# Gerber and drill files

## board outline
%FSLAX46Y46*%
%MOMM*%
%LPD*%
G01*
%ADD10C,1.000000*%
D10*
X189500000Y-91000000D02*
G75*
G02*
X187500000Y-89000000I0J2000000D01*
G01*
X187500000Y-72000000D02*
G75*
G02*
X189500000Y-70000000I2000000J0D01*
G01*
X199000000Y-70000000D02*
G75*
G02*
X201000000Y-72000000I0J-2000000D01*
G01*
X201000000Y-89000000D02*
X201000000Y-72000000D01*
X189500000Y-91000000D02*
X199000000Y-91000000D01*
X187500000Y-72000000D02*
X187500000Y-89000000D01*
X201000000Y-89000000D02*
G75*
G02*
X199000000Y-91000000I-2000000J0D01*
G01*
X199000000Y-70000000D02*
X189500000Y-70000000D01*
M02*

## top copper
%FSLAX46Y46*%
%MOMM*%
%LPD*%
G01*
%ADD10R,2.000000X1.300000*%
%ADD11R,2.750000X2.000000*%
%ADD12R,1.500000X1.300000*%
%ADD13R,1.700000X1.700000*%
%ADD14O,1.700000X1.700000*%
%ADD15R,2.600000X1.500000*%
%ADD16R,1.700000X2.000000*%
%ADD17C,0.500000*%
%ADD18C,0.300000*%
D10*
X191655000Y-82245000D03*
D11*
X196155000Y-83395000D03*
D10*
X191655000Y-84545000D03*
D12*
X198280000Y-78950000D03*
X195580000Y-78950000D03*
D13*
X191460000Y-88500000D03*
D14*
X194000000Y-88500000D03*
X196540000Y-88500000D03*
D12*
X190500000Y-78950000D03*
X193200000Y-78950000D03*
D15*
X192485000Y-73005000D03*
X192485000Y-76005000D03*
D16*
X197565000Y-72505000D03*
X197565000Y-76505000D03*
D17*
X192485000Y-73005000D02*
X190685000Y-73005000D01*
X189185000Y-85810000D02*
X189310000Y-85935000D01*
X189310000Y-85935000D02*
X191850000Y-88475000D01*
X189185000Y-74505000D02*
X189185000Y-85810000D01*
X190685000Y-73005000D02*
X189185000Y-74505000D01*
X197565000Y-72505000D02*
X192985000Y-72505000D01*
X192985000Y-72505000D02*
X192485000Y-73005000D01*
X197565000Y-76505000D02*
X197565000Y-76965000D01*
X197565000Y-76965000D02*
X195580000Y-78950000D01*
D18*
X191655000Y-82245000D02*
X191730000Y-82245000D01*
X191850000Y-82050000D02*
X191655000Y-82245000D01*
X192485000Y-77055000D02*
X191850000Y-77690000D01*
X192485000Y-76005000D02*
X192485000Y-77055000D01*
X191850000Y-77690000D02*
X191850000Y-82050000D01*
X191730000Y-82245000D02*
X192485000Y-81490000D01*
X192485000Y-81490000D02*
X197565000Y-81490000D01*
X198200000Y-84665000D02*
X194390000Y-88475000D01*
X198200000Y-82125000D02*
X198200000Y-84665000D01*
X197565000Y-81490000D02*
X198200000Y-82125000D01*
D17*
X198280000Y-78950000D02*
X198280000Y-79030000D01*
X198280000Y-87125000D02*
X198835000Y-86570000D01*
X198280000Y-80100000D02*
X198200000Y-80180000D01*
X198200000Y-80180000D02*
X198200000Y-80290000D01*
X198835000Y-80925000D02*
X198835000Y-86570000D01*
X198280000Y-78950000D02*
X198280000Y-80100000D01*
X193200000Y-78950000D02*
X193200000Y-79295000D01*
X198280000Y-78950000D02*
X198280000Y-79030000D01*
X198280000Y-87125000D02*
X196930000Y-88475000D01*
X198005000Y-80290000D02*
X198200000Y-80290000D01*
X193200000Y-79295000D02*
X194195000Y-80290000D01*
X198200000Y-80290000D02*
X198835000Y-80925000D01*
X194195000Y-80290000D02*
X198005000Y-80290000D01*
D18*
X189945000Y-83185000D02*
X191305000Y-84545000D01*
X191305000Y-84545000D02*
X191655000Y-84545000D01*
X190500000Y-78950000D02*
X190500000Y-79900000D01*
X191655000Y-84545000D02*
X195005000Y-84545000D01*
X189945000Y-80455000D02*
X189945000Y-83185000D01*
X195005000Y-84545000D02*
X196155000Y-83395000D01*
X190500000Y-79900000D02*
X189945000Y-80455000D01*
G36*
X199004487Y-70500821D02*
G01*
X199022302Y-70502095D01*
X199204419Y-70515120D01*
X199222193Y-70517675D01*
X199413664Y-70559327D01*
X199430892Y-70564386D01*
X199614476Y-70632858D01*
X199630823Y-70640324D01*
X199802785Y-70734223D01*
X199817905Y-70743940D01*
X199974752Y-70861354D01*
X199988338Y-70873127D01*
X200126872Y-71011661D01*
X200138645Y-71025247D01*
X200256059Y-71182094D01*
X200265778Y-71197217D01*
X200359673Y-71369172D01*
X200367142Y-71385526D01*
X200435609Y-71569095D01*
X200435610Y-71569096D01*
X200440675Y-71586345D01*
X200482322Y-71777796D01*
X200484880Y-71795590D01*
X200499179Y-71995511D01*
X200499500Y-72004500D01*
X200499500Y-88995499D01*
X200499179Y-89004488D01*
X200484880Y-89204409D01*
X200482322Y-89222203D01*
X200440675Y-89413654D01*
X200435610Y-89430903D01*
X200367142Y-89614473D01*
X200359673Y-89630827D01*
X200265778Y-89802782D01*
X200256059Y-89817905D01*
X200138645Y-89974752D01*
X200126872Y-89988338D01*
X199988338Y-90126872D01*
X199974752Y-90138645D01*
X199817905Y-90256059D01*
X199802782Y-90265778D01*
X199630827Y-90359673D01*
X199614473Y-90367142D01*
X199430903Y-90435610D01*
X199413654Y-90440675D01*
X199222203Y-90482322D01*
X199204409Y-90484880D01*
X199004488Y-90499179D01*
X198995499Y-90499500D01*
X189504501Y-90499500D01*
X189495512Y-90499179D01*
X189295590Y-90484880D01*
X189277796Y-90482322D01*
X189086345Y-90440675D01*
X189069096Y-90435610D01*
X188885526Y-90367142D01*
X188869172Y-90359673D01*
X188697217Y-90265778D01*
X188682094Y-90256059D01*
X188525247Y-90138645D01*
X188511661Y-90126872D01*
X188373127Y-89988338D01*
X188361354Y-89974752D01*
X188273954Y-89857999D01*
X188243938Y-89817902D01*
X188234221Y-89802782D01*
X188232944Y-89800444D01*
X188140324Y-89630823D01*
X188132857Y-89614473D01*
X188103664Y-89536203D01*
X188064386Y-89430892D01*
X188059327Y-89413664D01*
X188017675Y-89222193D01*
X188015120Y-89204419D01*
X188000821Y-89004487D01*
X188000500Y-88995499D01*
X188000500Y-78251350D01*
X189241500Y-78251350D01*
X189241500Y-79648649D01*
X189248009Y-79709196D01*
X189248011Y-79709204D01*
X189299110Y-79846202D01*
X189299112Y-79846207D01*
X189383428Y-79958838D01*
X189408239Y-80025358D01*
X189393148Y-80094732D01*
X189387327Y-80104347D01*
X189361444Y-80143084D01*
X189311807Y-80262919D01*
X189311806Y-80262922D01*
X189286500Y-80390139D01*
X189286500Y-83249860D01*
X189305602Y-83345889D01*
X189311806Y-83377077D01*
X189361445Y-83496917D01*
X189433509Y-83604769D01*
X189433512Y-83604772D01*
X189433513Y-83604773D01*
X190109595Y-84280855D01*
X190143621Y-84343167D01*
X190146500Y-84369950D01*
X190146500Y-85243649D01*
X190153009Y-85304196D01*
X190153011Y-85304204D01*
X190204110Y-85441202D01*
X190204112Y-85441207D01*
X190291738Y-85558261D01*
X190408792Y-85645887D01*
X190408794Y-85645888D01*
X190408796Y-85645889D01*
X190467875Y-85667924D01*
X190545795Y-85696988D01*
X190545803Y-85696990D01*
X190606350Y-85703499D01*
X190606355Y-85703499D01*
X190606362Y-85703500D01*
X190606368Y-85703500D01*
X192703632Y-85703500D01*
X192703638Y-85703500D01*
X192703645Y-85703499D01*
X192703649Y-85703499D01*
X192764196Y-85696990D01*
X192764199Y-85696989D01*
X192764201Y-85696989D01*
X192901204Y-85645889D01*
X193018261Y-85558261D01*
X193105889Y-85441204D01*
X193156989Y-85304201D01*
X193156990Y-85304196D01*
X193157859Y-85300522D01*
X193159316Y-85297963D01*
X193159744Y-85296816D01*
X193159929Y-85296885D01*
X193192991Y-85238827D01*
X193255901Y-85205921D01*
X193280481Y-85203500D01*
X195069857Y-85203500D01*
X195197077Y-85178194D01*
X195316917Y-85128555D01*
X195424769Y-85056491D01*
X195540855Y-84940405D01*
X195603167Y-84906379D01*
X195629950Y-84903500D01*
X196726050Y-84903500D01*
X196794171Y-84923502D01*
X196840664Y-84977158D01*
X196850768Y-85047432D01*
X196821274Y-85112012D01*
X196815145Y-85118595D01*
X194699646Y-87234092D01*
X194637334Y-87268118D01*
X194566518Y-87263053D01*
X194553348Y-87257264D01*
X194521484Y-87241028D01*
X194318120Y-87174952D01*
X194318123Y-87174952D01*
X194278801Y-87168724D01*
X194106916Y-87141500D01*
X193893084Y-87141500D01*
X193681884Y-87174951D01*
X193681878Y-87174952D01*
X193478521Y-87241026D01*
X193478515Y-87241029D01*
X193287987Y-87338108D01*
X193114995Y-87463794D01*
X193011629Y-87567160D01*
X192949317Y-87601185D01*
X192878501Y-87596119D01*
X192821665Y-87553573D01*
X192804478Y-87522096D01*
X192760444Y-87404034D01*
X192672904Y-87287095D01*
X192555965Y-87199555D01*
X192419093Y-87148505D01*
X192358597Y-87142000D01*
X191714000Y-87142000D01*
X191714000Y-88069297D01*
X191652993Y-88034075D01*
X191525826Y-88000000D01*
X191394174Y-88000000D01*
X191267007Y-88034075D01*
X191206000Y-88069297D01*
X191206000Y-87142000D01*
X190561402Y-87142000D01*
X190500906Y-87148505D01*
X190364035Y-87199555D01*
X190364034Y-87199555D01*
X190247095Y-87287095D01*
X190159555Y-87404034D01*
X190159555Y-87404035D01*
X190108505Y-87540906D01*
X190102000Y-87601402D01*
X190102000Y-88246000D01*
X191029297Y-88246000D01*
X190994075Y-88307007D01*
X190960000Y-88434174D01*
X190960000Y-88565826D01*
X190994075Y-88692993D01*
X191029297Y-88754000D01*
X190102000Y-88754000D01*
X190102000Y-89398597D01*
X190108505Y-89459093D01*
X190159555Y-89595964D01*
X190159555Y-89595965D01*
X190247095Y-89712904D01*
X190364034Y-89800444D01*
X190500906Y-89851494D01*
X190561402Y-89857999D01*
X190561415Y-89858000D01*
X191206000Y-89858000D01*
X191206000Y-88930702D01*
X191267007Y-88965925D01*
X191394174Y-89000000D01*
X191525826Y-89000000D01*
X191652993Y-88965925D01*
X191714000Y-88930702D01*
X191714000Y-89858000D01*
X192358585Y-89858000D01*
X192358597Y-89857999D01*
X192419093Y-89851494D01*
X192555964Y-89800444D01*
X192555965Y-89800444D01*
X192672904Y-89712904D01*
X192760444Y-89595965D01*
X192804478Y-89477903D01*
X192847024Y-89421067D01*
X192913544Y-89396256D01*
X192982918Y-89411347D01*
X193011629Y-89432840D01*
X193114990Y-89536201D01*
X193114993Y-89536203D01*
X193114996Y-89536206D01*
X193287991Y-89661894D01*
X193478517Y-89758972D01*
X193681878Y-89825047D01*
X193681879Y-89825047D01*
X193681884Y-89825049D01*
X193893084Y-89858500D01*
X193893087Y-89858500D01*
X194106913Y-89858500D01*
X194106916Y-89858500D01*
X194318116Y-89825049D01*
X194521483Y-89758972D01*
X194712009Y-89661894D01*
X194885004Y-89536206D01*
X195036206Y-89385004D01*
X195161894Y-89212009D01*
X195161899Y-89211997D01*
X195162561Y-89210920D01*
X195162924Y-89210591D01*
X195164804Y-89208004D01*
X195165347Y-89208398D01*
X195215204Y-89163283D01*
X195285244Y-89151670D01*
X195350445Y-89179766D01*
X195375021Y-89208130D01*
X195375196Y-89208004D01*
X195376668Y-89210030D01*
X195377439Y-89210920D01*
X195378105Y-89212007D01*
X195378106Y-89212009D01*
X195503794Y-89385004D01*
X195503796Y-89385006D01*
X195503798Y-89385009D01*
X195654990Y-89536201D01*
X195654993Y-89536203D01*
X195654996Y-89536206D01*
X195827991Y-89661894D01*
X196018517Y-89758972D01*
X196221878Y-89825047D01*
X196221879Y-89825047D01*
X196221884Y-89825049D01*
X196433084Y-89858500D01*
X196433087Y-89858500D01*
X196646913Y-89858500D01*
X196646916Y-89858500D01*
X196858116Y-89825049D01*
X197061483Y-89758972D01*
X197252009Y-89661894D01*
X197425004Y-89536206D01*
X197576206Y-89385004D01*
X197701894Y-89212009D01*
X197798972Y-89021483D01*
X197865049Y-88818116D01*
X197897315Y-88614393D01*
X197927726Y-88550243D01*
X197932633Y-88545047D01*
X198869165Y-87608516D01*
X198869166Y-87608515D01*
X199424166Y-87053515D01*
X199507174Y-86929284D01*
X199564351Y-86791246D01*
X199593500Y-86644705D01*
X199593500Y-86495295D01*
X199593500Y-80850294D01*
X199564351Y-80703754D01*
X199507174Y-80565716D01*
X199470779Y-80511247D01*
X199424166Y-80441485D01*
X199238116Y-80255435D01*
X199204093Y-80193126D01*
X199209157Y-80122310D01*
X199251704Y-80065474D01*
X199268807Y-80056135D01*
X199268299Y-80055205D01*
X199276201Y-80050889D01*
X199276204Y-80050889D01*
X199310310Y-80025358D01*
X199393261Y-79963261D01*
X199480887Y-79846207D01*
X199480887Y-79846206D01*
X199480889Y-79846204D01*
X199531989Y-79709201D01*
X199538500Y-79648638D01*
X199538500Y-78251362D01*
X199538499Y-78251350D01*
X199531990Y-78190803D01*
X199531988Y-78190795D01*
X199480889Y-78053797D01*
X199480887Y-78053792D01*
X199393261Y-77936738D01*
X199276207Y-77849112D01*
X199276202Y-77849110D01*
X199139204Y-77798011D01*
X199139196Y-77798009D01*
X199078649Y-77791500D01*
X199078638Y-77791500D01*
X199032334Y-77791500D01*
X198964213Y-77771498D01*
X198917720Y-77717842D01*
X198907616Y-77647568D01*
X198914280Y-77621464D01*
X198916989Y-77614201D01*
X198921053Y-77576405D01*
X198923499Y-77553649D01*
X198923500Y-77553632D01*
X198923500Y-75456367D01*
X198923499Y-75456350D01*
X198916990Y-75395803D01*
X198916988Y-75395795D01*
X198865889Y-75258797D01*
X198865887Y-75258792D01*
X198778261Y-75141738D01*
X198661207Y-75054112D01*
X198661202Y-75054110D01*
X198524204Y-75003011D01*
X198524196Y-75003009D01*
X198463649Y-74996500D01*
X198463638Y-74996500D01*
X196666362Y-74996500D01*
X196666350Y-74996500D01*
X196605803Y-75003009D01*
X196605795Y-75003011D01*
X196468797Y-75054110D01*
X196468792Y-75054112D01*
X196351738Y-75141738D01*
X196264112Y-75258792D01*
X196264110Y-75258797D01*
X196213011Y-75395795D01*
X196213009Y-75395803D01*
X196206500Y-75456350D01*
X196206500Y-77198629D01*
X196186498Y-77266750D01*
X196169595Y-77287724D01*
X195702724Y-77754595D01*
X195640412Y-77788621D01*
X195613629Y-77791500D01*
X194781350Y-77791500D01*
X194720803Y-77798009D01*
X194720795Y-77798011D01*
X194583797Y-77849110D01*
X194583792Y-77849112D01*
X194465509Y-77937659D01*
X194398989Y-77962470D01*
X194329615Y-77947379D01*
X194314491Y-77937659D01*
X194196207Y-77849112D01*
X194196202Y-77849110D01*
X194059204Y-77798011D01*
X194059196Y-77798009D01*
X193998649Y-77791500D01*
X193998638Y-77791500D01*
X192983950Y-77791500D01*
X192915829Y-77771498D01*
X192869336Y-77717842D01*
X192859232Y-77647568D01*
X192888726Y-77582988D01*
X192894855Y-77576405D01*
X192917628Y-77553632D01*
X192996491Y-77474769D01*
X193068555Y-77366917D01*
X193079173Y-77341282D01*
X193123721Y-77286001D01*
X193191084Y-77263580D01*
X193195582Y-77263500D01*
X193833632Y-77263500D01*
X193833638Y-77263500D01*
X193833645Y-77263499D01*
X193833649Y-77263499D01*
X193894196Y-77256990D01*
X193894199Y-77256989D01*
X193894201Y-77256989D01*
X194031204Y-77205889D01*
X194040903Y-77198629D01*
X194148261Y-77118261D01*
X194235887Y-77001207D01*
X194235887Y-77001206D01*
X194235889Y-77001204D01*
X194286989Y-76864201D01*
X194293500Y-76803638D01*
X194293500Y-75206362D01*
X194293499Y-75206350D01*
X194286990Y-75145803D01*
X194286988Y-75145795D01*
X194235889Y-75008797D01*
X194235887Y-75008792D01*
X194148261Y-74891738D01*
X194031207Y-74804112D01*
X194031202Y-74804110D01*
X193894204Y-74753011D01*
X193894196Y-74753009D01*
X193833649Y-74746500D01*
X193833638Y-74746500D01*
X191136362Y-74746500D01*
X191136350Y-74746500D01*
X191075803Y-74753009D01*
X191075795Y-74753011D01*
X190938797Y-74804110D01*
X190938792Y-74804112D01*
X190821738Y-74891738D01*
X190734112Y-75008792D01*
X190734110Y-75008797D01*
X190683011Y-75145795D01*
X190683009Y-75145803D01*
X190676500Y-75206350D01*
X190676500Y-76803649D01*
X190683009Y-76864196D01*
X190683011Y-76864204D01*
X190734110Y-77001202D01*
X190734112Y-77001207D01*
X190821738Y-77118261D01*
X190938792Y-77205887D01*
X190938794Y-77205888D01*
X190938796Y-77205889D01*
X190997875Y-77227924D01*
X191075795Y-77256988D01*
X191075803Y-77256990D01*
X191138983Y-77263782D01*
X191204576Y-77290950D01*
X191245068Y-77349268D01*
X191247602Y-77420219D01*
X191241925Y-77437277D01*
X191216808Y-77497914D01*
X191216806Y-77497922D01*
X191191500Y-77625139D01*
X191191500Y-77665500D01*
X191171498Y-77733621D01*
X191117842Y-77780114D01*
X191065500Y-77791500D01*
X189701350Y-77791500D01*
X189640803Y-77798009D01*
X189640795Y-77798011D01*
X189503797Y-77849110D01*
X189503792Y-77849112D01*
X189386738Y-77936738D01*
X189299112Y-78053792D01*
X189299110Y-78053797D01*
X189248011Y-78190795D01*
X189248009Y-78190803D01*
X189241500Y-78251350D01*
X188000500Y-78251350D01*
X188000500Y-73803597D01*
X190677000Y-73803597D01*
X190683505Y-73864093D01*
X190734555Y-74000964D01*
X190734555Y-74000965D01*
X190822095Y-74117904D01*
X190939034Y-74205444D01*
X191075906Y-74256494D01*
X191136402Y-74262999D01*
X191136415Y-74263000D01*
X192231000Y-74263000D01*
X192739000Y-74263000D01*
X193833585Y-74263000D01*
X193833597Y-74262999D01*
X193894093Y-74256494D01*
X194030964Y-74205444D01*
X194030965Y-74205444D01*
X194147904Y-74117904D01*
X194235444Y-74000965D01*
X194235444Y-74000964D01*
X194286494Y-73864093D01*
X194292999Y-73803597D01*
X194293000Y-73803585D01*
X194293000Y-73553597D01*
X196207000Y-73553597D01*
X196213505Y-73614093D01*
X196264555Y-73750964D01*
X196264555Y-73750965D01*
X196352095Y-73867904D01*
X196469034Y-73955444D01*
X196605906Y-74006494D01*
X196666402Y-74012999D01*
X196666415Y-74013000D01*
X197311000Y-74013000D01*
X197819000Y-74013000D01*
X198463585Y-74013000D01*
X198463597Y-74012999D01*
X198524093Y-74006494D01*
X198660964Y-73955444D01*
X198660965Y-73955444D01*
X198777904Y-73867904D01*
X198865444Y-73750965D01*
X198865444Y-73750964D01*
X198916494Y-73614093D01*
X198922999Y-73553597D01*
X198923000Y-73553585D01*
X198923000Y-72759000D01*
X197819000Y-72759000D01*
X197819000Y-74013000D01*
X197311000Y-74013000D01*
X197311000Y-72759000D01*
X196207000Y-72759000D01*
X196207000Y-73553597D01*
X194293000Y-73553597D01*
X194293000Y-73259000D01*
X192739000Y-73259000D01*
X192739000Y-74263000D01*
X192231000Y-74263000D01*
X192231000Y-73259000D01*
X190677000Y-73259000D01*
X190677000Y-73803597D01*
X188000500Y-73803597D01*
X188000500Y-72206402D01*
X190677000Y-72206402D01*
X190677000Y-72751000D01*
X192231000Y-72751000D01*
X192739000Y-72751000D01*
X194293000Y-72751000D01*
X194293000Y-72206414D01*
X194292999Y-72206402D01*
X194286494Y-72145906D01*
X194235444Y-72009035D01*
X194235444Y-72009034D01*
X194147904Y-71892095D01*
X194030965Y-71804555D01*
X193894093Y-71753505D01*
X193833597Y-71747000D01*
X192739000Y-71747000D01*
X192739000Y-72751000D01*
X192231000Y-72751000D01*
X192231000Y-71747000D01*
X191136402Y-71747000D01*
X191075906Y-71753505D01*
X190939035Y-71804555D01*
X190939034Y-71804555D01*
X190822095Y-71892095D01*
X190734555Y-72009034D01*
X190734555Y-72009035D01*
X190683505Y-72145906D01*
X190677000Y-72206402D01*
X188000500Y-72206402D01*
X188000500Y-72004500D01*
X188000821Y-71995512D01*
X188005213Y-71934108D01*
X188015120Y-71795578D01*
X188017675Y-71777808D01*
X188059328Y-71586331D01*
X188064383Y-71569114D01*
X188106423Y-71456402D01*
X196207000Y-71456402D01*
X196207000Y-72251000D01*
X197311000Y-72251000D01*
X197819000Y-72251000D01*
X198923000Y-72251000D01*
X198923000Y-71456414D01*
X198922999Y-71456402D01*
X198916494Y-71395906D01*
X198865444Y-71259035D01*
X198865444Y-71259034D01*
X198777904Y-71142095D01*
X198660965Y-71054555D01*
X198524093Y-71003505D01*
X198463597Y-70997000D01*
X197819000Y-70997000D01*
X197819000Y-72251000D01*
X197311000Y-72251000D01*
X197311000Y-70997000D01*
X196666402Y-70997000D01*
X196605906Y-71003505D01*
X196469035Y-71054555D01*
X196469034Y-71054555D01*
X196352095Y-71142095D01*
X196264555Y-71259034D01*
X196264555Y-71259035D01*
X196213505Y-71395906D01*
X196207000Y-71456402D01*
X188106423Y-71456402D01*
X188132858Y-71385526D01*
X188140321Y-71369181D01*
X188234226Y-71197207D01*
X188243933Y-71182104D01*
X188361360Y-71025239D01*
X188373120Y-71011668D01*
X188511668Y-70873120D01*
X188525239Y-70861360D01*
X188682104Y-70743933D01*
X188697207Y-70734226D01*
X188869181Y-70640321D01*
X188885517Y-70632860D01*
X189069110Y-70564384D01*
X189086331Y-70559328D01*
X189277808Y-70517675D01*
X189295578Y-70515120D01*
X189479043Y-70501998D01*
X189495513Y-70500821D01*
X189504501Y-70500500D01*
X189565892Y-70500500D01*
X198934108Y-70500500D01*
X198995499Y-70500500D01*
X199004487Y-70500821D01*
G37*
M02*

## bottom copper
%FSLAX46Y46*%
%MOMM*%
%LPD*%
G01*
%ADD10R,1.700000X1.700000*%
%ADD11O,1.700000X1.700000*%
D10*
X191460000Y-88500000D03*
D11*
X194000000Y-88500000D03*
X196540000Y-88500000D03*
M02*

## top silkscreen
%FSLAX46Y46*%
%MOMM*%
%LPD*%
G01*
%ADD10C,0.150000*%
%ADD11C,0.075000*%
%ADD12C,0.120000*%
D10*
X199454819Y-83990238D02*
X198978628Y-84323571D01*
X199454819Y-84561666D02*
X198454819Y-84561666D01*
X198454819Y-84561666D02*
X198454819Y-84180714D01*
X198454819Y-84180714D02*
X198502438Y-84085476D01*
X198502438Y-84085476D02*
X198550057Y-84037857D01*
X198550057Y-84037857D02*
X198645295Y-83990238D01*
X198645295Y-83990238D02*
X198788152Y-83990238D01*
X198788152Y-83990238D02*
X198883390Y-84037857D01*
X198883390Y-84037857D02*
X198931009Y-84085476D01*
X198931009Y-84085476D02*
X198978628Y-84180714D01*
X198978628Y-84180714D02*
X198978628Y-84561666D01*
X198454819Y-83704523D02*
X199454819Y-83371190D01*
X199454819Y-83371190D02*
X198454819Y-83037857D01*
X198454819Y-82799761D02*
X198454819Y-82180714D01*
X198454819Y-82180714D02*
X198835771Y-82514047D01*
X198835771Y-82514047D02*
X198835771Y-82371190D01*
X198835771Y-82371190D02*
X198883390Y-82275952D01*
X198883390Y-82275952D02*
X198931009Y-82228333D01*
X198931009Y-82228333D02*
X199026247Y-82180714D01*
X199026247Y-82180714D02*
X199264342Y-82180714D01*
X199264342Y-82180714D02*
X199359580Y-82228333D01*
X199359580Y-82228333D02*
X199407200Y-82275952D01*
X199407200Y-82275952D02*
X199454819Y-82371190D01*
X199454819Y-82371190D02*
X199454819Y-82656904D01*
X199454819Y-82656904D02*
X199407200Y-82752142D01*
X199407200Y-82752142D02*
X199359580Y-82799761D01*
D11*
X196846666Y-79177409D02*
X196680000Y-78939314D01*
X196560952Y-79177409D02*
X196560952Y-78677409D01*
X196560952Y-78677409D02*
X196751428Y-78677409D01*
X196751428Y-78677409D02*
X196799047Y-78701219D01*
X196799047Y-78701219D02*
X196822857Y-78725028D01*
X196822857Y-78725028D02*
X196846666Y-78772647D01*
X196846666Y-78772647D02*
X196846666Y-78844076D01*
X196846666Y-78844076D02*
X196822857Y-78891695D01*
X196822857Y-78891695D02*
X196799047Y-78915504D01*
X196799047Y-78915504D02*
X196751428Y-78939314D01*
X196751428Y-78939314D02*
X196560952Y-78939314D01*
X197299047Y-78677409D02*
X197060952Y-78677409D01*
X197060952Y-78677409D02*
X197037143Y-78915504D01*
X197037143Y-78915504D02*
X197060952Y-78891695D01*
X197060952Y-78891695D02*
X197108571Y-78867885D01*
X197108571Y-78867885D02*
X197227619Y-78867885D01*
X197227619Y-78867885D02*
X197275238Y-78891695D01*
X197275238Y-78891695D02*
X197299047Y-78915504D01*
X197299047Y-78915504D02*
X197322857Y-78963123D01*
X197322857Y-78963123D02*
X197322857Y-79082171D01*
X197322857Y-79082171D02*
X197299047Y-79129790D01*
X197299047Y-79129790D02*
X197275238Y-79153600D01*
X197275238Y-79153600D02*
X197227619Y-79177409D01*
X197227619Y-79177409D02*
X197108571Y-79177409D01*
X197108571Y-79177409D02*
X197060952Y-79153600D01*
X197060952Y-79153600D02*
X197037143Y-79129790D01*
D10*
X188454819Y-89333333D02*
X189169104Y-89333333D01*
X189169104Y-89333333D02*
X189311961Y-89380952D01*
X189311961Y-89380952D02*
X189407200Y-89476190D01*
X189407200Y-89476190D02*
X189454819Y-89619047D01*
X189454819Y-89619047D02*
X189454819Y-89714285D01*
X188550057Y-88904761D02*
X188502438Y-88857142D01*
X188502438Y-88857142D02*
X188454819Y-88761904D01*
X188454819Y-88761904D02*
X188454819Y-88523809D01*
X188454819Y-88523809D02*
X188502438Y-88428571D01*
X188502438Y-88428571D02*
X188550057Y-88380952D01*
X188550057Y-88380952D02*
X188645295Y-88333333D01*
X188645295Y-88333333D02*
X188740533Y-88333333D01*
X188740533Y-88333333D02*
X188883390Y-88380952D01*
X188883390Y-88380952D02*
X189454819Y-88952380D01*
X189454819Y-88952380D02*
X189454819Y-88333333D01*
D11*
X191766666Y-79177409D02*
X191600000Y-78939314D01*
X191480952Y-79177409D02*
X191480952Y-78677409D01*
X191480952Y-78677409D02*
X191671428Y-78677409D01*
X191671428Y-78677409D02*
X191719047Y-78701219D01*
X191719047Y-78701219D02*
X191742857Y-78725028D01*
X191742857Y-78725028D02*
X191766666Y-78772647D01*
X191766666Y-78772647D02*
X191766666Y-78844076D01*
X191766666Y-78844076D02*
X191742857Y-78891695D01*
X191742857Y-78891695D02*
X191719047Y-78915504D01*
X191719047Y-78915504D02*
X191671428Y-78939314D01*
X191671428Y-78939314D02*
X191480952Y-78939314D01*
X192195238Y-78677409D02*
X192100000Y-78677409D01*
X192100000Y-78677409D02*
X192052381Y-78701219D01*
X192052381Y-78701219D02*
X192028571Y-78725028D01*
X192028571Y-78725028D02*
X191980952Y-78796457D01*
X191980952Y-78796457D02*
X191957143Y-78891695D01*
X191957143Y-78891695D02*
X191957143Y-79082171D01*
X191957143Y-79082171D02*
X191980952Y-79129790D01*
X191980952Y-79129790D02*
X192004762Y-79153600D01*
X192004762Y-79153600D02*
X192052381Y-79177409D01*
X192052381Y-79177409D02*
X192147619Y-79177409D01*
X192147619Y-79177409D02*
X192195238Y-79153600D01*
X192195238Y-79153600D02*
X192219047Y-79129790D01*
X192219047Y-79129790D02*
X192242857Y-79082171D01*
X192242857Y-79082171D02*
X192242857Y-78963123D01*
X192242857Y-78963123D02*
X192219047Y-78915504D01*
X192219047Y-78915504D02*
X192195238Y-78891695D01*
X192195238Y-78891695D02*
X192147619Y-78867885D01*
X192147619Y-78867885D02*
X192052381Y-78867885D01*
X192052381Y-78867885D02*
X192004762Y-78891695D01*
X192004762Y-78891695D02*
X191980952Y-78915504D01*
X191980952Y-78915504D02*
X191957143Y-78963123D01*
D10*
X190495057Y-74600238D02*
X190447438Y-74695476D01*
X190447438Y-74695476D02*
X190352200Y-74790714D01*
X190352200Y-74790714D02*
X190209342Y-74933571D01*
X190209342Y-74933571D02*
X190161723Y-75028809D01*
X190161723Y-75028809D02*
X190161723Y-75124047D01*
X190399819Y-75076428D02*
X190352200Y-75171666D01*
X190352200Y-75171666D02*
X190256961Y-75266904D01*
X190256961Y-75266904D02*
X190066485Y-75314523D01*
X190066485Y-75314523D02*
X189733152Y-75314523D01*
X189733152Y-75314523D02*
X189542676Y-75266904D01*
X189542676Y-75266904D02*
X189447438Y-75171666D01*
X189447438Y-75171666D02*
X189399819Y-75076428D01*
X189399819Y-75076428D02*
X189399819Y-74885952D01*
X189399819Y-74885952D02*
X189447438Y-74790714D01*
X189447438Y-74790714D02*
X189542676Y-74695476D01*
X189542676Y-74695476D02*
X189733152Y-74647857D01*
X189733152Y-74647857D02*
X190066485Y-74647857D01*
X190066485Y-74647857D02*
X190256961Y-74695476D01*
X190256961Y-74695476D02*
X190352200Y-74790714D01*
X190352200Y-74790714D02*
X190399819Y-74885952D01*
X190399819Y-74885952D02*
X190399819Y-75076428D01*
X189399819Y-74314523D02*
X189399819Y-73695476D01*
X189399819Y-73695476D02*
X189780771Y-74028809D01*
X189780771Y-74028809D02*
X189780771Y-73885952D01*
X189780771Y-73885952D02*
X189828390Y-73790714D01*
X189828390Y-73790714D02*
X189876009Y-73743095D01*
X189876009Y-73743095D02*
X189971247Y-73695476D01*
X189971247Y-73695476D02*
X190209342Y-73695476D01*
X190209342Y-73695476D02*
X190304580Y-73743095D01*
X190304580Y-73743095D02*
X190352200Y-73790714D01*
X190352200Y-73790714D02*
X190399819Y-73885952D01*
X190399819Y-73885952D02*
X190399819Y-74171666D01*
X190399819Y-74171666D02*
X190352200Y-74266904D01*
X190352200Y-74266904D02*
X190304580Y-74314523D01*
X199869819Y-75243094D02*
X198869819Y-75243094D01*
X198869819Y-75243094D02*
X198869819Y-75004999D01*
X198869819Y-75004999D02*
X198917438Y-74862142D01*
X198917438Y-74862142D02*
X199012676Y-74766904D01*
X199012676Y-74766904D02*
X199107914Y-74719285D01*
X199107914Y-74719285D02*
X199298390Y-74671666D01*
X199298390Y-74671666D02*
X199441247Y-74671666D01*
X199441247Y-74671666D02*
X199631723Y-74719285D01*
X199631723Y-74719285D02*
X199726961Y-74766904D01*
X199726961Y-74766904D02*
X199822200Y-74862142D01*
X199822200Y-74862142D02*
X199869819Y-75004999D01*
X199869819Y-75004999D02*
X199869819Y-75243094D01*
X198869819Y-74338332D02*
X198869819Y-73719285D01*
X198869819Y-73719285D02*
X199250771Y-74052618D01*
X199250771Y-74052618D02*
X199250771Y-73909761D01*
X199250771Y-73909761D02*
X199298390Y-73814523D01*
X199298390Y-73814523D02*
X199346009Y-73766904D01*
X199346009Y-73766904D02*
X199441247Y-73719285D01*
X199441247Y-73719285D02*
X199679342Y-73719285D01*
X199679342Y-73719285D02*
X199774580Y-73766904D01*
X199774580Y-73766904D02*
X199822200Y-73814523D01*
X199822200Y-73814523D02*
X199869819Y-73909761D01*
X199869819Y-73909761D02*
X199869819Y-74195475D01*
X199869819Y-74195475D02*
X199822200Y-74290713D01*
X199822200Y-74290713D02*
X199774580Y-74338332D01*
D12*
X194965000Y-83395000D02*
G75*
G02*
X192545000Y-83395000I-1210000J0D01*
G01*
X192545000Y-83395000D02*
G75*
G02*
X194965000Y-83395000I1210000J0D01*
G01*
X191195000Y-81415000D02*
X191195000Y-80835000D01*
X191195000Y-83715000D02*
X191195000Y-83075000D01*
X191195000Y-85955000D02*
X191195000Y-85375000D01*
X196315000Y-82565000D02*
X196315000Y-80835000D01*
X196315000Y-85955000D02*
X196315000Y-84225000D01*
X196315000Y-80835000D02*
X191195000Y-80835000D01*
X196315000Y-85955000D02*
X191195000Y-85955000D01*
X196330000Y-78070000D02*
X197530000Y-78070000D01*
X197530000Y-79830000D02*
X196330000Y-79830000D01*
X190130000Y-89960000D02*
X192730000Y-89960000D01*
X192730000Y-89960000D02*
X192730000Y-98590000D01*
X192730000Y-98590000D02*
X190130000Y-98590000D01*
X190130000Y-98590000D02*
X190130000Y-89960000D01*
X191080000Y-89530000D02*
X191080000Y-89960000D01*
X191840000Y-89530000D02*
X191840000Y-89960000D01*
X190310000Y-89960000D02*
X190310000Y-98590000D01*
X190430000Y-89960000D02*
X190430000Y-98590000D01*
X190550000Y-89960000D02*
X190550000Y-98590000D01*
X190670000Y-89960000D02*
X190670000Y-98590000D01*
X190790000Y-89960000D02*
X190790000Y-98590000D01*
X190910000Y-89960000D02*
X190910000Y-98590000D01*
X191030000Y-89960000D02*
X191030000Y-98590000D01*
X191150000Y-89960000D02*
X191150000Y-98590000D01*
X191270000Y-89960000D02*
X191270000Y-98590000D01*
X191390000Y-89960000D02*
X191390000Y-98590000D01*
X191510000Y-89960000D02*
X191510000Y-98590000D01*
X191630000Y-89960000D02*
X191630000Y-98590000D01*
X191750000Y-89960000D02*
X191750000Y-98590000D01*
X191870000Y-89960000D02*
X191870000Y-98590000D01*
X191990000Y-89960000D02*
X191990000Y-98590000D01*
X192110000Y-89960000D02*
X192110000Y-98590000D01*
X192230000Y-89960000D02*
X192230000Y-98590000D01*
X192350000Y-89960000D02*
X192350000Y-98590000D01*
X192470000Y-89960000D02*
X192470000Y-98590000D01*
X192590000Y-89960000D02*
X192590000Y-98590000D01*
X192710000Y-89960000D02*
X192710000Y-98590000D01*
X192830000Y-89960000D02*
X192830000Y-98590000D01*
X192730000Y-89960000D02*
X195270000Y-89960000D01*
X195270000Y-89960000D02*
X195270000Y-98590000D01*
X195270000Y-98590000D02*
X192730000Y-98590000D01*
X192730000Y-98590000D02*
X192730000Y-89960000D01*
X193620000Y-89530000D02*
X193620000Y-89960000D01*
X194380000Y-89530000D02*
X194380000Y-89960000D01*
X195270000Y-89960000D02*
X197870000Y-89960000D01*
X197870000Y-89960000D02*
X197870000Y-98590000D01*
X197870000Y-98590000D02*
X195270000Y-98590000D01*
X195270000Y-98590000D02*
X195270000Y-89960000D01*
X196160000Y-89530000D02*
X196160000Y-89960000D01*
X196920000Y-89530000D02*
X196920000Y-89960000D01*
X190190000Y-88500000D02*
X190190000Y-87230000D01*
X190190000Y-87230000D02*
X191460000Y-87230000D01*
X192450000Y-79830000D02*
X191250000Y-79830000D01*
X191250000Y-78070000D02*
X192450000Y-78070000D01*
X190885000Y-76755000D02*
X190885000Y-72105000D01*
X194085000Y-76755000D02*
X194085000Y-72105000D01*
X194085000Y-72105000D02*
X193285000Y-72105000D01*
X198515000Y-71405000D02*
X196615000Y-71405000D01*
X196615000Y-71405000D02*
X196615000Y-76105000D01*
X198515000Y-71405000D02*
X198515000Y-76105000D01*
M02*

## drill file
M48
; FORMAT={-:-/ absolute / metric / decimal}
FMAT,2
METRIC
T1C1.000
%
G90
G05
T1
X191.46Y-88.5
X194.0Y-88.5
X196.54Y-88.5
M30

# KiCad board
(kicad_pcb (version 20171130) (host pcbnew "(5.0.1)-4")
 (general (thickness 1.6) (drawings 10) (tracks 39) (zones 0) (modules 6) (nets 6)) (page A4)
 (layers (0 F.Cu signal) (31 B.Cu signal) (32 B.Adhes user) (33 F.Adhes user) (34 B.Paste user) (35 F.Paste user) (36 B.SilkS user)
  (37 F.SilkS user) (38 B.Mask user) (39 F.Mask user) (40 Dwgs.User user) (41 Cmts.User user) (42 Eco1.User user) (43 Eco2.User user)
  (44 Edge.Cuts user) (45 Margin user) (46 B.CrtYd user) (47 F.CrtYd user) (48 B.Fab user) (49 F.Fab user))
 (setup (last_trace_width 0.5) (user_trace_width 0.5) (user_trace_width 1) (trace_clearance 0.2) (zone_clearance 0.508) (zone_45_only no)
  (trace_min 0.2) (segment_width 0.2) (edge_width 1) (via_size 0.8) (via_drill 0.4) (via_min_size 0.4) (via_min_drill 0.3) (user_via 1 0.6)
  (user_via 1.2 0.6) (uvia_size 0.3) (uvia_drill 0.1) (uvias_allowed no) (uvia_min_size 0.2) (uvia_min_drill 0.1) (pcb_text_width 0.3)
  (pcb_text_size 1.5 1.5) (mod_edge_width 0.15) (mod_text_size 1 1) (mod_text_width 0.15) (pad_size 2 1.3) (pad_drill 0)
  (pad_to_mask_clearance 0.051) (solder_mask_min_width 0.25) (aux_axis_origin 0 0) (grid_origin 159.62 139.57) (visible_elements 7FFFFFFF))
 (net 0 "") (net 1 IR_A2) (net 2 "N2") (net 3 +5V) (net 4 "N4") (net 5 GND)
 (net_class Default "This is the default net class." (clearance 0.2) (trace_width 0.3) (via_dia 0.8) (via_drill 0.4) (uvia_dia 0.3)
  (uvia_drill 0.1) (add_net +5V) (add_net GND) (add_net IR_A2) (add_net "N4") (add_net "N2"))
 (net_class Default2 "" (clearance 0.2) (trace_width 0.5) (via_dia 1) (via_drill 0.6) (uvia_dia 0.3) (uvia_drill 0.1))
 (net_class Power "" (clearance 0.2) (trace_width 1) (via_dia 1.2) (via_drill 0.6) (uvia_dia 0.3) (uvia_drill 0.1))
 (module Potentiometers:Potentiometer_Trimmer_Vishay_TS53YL (layer F.Cu) (at 193.755 83.395 180)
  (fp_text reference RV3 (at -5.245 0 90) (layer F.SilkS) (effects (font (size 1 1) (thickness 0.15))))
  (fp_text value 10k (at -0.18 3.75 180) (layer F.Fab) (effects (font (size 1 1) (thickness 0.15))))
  (fp_circle (center 0 0) (end 1.21 0) (layer F.SilkS) (width 0.12))
  (fp_line (start 2.56 1.98) (end 2.56 2.56) (layer F.SilkS) (width 0.12))
  (fp_line (start 2.56 -0.32) (end 2.56 0.32) (layer F.SilkS) (width 0.12))
  (fp_line (start 2.56 -2.56) (end 2.56 -1.98) (layer F.SilkS) (width 0.12))
  (fp_line (start -2.56 0.83) (end -2.56 2.56) (layer F.SilkS) (width 0.12))
  (fp_line (start -2.56 -2.56) (end -2.56 -0.83) (layer F.SilkS) (width 0.12))
  (fp_line (start -2.56 2.56) (end 2.56 2.56) (layer F.SilkS) (width 0.12))
  (fp_line (start -2.56 -2.56) (end 2.56 -2.56) (layer F.SilkS) (width 0.12))
  (pad 3 smd rect (at 2.1 1.15 180) (size 2 1.3) (layers F.Cu F.Mask) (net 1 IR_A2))
  (pad 2 smd rect (at -2.4 0 180) (size 2.75 2) (layers F.Cu F.Mask) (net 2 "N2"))
  (pad 1 smd rect (at 2.1 -1.15 180) (size 2 1.3) (layers F.Cu F.Mask) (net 2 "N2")))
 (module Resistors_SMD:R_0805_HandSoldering (layer F.Cu) (at 196.93 78.95 180)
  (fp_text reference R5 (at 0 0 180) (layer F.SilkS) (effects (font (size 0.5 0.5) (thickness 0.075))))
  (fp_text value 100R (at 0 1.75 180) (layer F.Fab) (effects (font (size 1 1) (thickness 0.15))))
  (fp_line (start 0.6 0.88) (end -0.6 0.88) (layer F.SilkS) (width 0.12))
  (fp_line (start -0.6 -0.88) (end 0.6 -0.88) (layer F.SilkS) (width 0.12))
  (pad 1 smd rect (at -1.35 0 180) (size 1.5 1.3) (layers F.Cu F.Paste F.Mask) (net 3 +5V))
  (pad 2 smd rect (at 1.35 0 180) (size 1.5 1.3) (layers F.Cu F.Paste F.Mask) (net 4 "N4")))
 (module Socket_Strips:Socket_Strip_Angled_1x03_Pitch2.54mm (layer F.Cu) (at 191.46 88.5 90)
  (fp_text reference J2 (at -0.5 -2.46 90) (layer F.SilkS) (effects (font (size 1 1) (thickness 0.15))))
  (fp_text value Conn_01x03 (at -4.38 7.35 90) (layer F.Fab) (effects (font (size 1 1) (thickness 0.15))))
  (fp_line (start -1.46 -1.33) (end -1.46 1.27) (layer F.SilkS) (width 0.12))
  (fp_line (start -1.46 1.27) (end -10.09 1.27) (layer F.SilkS) (width 0.12))
  (fp_line (start -10.09 1.27) (end -10.09 -1.33) (layer F.SilkS) (width 0.12))
  (fp_line (start -10.09 -1.33) (end -1.46 -1.33) (layer F.SilkS) (width 0.12))
  (fp_line (start -1.03 -0.38) (end -1.46 -0.38) (layer F.SilkS) (width 0.12))
  (fp_line (start -1.03 0.38) (end -1.46 0.38) (layer F.SilkS) (width 0.12))
  (fp_line (start -1.46 -1.15) (end -10.09 -1.15) (layer F.SilkS) (width 0.12))
  (fp_line (start -1.46 -1.03) (end -10.09 -1.03) (layer F.SilkS) (width 0.12))
  (fp_line (start -1.46 -0.91) (end -10.09 -0.91) (layer F.SilkS) (width 0.12))
  (fp_line (start -1.46 -0.79) (end -10.09 -0.79) (layer F.SilkS) (width 0.12))
  (fp_line (start -1.46 -0.67) (end -10.09 -0.67) (layer F.SilkS) (width 0.12))
  (fp_line (start -1.46 -0.55) (end -10.09 -0.55) (layer F.SilkS) (width 0.12))
  (fp_line (start -1.46 -0.43) (end -10.09 -0.43) (layer F.SilkS) (width 0.12))
  (fp_line (start -1.46 -0.31) (end -10.09 -0.31) (layer F.SilkS) (width 0.12))
  (fp_line (start -1.46 -0.19) (end -10.09 -0.19) (layer F.SilkS) (width 0.12))
  (fp_line (start -1.46 -0.07) (end -10.09 -0.07) (layer F.SilkS) (width 0.12))
  (fp_line (start -1.46 0.05) (end -10.09 0.05) (layer F.SilkS) (width 0.12))
  (fp_line (start -1.46 0.17) (end -10.09 0.17) (layer F.SilkS) (width 0.12))
  (fp_line (start -1.46 0.29) (end -10.09 0.29) (layer F.SilkS) (width 0.12))
  (fp_line (start -1.46 0.41) (end -10.09 0.41) (layer F.SilkS) (width 0.12))
  (fp_line (start -1.46 0.53) (end -10.09 0.53) (layer F.SilkS) (width 0.12))
  (fp_line (start -1.46 0.65) (end -10.09 0.65) (layer F.SilkS) (width 0.12))
  (fp_line (start -1.46 0.77) (end -10.09 0.77) (layer F.SilkS) (width 0.12))
  (fp_line (start -1.46 0.89) (end -10.09 0.89) (layer F.SilkS) (width 0.12))
  (fp_line (start -1.46 1.01) (end -10.09 1.01) (layer F.SilkS) (width 0.12))
  (fp_line (start -1.46 1.13) (end -10.09 1.13) (layer F.SilkS) (width 0.12))
  (fp_line (start -1.46 1.25) (end -10.09 1.25) (layer F.SilkS) (width 0.12))
  (fp_line (start -1.46 1.37) (end -10.09 1.37) (layer F.SilkS) (width 0.12))
  (fp_line (start -1.46 1.27) (end -1.46 3.81) (layer F.SilkS) (width 0.12))
  (fp_line (start -1.46 3.81) (end -10.09 3.81) (layer F.SilkS) (width 0.12))
  (fp_line (start -10.09 3.81) (end -10.09 1.27) (layer F.SilkS) (width 0.12))
  (fp_line (start -10.09 1.27) (end -1.46 1.27) (layer F.SilkS) (width 0.12))
  (fp_line (start -1.03 2.16) (end -1.46 2.16) (layer F.SilkS) (width 0.12))
  (fp_line (start -1.03 2.92) (end -1.46 2.92) (layer F.SilkS) (width 0.12))
  (fp_line (start -1.46 3.81) (end -1.46 6.41) (layer F.SilkS) (width 0.12))
  (fp_line (start -1.46 6.41) (end -10.09 6.41) (layer F.SilkS) (width 0.12))
  (fp_line (start -10.09 6.41) (end -10.09 3.81) (layer F.SilkS) (width 0.12))
  (fp_line (start -10.09 3.81) (end -1.46 3.81) (layer F.SilkS) (width 0.12))
  (fp_line (start -1.03 4.7) (end -1.46 4.7) (layer F.SilkS) (width 0.12))
  (fp_line (start -1.03 5.46) (end -1.46 5.46) (layer F.SilkS) (width 0.12))
  (fp_line (start 0 -1.27) (end 1.27 -1.27) (layer F.SilkS) (width 0.12))
  (fp_line (start 1.27 -1.27) (end 1.27 0) (layer F.SilkS) (width 0.12))
  (pad 1 thru_hole rect (at 0 0 90) (size 1.7 1.7) (drill 1) (layers *.Cu *.Mask) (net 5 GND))
  (pad 2 thru_hole oval (at 0 2.54 90) (size 1.7 1.7) (drill 1) (layers *.Cu *.Mask) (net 1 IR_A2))
  (pad 3 thru_hole oval (at 0 5.08 90) (size 1.7 1.7) (drill 1) (layers *.Cu *.Mask) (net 3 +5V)))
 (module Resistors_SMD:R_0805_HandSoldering (layer F.Cu) (at 191.85 78.95 180)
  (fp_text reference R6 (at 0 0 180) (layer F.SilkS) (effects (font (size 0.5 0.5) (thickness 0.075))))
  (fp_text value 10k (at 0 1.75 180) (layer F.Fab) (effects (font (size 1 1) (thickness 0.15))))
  (fp_line (start -0.6 -0.88) (end 0.6 -0.88) (layer F.SilkS) (width 0.12))
  (fp_line (start 0.6 0.88) (end -0.6 0.88) (layer F.SilkS) (width 0.12))
  (pad 2 smd rect (at 1.35 0 180) (size 1.5 1.3) (layers F.Cu F.Paste F.Mask) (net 2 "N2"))
  (pad 1 smd rect (at -1.35 0 180) (size 1.5 1.3) (layers F.Cu F.Paste F.Mask) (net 3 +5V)))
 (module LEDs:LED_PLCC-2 (layer F.Cu) (at 192.485 74.505 270)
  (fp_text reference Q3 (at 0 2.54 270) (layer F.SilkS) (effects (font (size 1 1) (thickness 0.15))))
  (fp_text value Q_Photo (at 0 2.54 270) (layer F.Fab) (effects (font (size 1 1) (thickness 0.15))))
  (fp_line (start 2.25 1.6) (end -2.4 1.6) (layer F.SilkS) (width 0.12))
  (fp_line (start 2.25 -1.6) (end -2.4 -1.6) (layer F.SilkS) (width 0.12))
  (fp_line (start -2.4 -1.6) (end -2.4 -0.8) (layer F.SilkS) (width 0.12))
  (pad 1 smd rect (at -1.5 0 270) (size 1.5 2.6) (layers F.Cu F.Paste F.Mask) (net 5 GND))
  (pad 2 smd rect (at 1.5 0 270) (size 1.5 2.6) (layers F.Cu F.Paste F.Mask) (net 1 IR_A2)))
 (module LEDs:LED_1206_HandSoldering (layer F.Cu) (at 197.565 74.505 270)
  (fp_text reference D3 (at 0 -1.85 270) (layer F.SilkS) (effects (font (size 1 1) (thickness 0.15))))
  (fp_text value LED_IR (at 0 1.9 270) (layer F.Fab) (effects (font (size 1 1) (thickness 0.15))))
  (fp_line (start -3.1 -0.95) (end -3.1 0.95) (layer F.SilkS) (width 0.12))
  (fp_line (start -3.1 0.95) (end 1.6 0.95) (layer F.SilkS) (width 0.12))
  (fp_line (start -3.1 -0.95) (end 1.6 -0.95) (layer F.SilkS) (width 0.12))
  (pad 1 smd rect (at -2 0 270) (size 2 1.7) (layers F.Cu F.Paste F.Mask) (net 5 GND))
  (pad 2 smd rect (at 2 0 270) (size 2 1.7) (layers F.Cu F.Paste F.Mask) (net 4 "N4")))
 (gr_arc (start 189.5 89) (end 187.5 89) (angle -90) (layer Edge.Cuts) (width 1))
 (gr_arc (start 189.5 72) (end 189.5 70) (angle -90) (layer Edge.Cuts) (width 1))
 (gr_arc (start 199 72) (end 201 72) (angle -90) (layer Edge.Cuts) (width 1))
 (gr_line (start 201 89) (end 201 72) (layer Edge.Cuts) (width 1))
 (gr_line (start 189.5 91) (end 199 91) (layer Edge.Cuts) (width 1))
 (gr_line (start 187.5 72) (end 187.5 89) (layer Edge.Cuts) (width 1))
 (gr_arc (start 199 89) (end 199 91) (angle -90) (layer Edge.Cuts) (width 1))
 (gr_line (start 199 70) (end 189.5 70) (layer Edge.Cuts) (width 1))
 (segment (start 192.485 73.005) (end 190.685 73.005) (width 0.5) (layer F.Cu) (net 5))
 (segment (start 189.185 85.81) (end 189.31 85.935) (width 0.5) (layer F.Cu) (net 5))
 (segment (start 189.31 85.935) (end 191.85 88.475) (width 0.5) (layer F.Cu) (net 5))
 (segment (start 189.185 74.505) (end 189.185 85.81) (width 0.5) (layer F.Cu) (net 5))
 (segment (start 190.685 73.005) (end 189.185 74.505) (width 0.5) (layer F.Cu) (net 5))
 (segment (start 197.565 72.505) (end 192.985 72.505) (width 0.5) (layer F.Cu) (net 5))
 (segment (start 192.985 72.505) (end 192.485 73.005) (width 0.5) (layer F.Cu) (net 5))
 (segment (start 197.565 76.505) (end 197.565 76.965) (width 0.5) (layer F.Cu) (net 4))
 (segment (start 197.565 76.965) (end 195.58 78.95) (width 0.5) (layer F.Cu) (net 4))
 (segment (start 191.655 82.245) (end 191.73 82.245) (width 0.3) (layer F.Cu) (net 1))
 (segment (start 191.85 82.05) (end 191.655 82.245) (width 0.3) (layer F.Cu) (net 1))
 (segment (start 192.485 77.055) (end 191.85 77.69) (width 0.3) (layer F.Cu) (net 1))
 (segment (start 192.485 76.005) (end 192.485 77.055) (width 0.3) (layer F.Cu) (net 1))
 (segment (start 191.85 77.69) (end 191.85 82.05) (width 0.3) (layer F.Cu) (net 1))
 (segment (start 191.73 82.245) (end 192.485 81.49) (width 0.3) (layer F.Cu) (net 1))
 (segment (start 192.485 81.49) (end 197.565 81.49) (width 0.3) (layer F.Cu) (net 1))
 (segment (start 198.2 84.665) (end 194.39 88.475) (width 0.3) (layer F.Cu) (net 1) (status 1000000))
 (segment (start 198.2 82.125) (end 198.2 84.665) (width 0.3) (layer F.Cu) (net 1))
 (segment (start 197.565 81.49) (end 198.2 82.125) (width 0.3) (layer F.Cu) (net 1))
 (segment (start 198.28 78.95) (end 198.28 79.03) (width 0.5) (layer F.Cu) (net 3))
 (segment (start 198.28 87.125) (end 198.835 86.57) (width 0.5) (layer F.Cu) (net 3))
 (segment (start 198.28 80.1) (end 198.2 80.18) (width 0.5) (layer F.Cu) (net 3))
 (segment (start 198.2 80.18) (end 198.2 80.29) (width 0.5) (layer F.Cu) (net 3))
 (segment (start 198.835 80.925) (end 198.835 86.57) (width 0.5) (layer F.Cu) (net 3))
 (segment (start 198.28 78.95) (end 198.28 80.1) (width 0.5) (layer F.Cu) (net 3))
 (segment (start 193.2 78.95) (end 193.2 79.295) (width 0.5) (layer F.Cu) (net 3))
 (segment (start 198.28 78.95) (end 198.28 79.03) (width 0.5) (layer F.Cu) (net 3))
 (segment (start 198.28 87.125) (end 196.93 88.475) (width 0.5) (layer F.Cu) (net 3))
 (segment (start 198.005 80.29) (end 198.2 80.29) (width 0.5) (layer F.Cu) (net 3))
 (segment (start 193.2 79.295) (end 194.195 80.29) (width 0.5) (layer F.Cu) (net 3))
 (segment (start 198.2 80.29) (end 198.835 80.925) (width 0.5) (layer F.Cu) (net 3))
 (segment (start 194.195 80.29) (end 198.005 80.29) (width 0.5) (layer F.Cu) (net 3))
 (segment (start 189.945 83.185) (end 191.305 84.545) (width 0.3) (layer F.Cu) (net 2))
 (segment (start 191.305 84.545) (end 191.655 84.545) (width 0.3) (layer F.Cu) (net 2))
 (segment (start 190.5 78.95) (end 190.5 79.9) (width 0.3) (layer F.Cu) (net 2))
 (segment (start 191.655 84.545) (end 195.005 84.545) (width 0.3) (layer F.Cu) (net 2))
 (segment (start 189.945 80.455) (end 189.945 83.185) (width 0.3) (layer F.Cu) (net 2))
 (segment (start 195.005 84.545) (end 196.155 83.395) (width 0.3) (layer F.Cu) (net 2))
 (segment (start 190.5 79.9) (end 189.945 80.455) (width 0.3) (layer F.Cu) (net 2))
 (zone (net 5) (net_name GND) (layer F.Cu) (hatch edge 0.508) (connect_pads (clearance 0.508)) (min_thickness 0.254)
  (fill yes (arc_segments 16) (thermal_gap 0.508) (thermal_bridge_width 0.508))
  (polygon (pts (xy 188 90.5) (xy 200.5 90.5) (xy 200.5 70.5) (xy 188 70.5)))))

